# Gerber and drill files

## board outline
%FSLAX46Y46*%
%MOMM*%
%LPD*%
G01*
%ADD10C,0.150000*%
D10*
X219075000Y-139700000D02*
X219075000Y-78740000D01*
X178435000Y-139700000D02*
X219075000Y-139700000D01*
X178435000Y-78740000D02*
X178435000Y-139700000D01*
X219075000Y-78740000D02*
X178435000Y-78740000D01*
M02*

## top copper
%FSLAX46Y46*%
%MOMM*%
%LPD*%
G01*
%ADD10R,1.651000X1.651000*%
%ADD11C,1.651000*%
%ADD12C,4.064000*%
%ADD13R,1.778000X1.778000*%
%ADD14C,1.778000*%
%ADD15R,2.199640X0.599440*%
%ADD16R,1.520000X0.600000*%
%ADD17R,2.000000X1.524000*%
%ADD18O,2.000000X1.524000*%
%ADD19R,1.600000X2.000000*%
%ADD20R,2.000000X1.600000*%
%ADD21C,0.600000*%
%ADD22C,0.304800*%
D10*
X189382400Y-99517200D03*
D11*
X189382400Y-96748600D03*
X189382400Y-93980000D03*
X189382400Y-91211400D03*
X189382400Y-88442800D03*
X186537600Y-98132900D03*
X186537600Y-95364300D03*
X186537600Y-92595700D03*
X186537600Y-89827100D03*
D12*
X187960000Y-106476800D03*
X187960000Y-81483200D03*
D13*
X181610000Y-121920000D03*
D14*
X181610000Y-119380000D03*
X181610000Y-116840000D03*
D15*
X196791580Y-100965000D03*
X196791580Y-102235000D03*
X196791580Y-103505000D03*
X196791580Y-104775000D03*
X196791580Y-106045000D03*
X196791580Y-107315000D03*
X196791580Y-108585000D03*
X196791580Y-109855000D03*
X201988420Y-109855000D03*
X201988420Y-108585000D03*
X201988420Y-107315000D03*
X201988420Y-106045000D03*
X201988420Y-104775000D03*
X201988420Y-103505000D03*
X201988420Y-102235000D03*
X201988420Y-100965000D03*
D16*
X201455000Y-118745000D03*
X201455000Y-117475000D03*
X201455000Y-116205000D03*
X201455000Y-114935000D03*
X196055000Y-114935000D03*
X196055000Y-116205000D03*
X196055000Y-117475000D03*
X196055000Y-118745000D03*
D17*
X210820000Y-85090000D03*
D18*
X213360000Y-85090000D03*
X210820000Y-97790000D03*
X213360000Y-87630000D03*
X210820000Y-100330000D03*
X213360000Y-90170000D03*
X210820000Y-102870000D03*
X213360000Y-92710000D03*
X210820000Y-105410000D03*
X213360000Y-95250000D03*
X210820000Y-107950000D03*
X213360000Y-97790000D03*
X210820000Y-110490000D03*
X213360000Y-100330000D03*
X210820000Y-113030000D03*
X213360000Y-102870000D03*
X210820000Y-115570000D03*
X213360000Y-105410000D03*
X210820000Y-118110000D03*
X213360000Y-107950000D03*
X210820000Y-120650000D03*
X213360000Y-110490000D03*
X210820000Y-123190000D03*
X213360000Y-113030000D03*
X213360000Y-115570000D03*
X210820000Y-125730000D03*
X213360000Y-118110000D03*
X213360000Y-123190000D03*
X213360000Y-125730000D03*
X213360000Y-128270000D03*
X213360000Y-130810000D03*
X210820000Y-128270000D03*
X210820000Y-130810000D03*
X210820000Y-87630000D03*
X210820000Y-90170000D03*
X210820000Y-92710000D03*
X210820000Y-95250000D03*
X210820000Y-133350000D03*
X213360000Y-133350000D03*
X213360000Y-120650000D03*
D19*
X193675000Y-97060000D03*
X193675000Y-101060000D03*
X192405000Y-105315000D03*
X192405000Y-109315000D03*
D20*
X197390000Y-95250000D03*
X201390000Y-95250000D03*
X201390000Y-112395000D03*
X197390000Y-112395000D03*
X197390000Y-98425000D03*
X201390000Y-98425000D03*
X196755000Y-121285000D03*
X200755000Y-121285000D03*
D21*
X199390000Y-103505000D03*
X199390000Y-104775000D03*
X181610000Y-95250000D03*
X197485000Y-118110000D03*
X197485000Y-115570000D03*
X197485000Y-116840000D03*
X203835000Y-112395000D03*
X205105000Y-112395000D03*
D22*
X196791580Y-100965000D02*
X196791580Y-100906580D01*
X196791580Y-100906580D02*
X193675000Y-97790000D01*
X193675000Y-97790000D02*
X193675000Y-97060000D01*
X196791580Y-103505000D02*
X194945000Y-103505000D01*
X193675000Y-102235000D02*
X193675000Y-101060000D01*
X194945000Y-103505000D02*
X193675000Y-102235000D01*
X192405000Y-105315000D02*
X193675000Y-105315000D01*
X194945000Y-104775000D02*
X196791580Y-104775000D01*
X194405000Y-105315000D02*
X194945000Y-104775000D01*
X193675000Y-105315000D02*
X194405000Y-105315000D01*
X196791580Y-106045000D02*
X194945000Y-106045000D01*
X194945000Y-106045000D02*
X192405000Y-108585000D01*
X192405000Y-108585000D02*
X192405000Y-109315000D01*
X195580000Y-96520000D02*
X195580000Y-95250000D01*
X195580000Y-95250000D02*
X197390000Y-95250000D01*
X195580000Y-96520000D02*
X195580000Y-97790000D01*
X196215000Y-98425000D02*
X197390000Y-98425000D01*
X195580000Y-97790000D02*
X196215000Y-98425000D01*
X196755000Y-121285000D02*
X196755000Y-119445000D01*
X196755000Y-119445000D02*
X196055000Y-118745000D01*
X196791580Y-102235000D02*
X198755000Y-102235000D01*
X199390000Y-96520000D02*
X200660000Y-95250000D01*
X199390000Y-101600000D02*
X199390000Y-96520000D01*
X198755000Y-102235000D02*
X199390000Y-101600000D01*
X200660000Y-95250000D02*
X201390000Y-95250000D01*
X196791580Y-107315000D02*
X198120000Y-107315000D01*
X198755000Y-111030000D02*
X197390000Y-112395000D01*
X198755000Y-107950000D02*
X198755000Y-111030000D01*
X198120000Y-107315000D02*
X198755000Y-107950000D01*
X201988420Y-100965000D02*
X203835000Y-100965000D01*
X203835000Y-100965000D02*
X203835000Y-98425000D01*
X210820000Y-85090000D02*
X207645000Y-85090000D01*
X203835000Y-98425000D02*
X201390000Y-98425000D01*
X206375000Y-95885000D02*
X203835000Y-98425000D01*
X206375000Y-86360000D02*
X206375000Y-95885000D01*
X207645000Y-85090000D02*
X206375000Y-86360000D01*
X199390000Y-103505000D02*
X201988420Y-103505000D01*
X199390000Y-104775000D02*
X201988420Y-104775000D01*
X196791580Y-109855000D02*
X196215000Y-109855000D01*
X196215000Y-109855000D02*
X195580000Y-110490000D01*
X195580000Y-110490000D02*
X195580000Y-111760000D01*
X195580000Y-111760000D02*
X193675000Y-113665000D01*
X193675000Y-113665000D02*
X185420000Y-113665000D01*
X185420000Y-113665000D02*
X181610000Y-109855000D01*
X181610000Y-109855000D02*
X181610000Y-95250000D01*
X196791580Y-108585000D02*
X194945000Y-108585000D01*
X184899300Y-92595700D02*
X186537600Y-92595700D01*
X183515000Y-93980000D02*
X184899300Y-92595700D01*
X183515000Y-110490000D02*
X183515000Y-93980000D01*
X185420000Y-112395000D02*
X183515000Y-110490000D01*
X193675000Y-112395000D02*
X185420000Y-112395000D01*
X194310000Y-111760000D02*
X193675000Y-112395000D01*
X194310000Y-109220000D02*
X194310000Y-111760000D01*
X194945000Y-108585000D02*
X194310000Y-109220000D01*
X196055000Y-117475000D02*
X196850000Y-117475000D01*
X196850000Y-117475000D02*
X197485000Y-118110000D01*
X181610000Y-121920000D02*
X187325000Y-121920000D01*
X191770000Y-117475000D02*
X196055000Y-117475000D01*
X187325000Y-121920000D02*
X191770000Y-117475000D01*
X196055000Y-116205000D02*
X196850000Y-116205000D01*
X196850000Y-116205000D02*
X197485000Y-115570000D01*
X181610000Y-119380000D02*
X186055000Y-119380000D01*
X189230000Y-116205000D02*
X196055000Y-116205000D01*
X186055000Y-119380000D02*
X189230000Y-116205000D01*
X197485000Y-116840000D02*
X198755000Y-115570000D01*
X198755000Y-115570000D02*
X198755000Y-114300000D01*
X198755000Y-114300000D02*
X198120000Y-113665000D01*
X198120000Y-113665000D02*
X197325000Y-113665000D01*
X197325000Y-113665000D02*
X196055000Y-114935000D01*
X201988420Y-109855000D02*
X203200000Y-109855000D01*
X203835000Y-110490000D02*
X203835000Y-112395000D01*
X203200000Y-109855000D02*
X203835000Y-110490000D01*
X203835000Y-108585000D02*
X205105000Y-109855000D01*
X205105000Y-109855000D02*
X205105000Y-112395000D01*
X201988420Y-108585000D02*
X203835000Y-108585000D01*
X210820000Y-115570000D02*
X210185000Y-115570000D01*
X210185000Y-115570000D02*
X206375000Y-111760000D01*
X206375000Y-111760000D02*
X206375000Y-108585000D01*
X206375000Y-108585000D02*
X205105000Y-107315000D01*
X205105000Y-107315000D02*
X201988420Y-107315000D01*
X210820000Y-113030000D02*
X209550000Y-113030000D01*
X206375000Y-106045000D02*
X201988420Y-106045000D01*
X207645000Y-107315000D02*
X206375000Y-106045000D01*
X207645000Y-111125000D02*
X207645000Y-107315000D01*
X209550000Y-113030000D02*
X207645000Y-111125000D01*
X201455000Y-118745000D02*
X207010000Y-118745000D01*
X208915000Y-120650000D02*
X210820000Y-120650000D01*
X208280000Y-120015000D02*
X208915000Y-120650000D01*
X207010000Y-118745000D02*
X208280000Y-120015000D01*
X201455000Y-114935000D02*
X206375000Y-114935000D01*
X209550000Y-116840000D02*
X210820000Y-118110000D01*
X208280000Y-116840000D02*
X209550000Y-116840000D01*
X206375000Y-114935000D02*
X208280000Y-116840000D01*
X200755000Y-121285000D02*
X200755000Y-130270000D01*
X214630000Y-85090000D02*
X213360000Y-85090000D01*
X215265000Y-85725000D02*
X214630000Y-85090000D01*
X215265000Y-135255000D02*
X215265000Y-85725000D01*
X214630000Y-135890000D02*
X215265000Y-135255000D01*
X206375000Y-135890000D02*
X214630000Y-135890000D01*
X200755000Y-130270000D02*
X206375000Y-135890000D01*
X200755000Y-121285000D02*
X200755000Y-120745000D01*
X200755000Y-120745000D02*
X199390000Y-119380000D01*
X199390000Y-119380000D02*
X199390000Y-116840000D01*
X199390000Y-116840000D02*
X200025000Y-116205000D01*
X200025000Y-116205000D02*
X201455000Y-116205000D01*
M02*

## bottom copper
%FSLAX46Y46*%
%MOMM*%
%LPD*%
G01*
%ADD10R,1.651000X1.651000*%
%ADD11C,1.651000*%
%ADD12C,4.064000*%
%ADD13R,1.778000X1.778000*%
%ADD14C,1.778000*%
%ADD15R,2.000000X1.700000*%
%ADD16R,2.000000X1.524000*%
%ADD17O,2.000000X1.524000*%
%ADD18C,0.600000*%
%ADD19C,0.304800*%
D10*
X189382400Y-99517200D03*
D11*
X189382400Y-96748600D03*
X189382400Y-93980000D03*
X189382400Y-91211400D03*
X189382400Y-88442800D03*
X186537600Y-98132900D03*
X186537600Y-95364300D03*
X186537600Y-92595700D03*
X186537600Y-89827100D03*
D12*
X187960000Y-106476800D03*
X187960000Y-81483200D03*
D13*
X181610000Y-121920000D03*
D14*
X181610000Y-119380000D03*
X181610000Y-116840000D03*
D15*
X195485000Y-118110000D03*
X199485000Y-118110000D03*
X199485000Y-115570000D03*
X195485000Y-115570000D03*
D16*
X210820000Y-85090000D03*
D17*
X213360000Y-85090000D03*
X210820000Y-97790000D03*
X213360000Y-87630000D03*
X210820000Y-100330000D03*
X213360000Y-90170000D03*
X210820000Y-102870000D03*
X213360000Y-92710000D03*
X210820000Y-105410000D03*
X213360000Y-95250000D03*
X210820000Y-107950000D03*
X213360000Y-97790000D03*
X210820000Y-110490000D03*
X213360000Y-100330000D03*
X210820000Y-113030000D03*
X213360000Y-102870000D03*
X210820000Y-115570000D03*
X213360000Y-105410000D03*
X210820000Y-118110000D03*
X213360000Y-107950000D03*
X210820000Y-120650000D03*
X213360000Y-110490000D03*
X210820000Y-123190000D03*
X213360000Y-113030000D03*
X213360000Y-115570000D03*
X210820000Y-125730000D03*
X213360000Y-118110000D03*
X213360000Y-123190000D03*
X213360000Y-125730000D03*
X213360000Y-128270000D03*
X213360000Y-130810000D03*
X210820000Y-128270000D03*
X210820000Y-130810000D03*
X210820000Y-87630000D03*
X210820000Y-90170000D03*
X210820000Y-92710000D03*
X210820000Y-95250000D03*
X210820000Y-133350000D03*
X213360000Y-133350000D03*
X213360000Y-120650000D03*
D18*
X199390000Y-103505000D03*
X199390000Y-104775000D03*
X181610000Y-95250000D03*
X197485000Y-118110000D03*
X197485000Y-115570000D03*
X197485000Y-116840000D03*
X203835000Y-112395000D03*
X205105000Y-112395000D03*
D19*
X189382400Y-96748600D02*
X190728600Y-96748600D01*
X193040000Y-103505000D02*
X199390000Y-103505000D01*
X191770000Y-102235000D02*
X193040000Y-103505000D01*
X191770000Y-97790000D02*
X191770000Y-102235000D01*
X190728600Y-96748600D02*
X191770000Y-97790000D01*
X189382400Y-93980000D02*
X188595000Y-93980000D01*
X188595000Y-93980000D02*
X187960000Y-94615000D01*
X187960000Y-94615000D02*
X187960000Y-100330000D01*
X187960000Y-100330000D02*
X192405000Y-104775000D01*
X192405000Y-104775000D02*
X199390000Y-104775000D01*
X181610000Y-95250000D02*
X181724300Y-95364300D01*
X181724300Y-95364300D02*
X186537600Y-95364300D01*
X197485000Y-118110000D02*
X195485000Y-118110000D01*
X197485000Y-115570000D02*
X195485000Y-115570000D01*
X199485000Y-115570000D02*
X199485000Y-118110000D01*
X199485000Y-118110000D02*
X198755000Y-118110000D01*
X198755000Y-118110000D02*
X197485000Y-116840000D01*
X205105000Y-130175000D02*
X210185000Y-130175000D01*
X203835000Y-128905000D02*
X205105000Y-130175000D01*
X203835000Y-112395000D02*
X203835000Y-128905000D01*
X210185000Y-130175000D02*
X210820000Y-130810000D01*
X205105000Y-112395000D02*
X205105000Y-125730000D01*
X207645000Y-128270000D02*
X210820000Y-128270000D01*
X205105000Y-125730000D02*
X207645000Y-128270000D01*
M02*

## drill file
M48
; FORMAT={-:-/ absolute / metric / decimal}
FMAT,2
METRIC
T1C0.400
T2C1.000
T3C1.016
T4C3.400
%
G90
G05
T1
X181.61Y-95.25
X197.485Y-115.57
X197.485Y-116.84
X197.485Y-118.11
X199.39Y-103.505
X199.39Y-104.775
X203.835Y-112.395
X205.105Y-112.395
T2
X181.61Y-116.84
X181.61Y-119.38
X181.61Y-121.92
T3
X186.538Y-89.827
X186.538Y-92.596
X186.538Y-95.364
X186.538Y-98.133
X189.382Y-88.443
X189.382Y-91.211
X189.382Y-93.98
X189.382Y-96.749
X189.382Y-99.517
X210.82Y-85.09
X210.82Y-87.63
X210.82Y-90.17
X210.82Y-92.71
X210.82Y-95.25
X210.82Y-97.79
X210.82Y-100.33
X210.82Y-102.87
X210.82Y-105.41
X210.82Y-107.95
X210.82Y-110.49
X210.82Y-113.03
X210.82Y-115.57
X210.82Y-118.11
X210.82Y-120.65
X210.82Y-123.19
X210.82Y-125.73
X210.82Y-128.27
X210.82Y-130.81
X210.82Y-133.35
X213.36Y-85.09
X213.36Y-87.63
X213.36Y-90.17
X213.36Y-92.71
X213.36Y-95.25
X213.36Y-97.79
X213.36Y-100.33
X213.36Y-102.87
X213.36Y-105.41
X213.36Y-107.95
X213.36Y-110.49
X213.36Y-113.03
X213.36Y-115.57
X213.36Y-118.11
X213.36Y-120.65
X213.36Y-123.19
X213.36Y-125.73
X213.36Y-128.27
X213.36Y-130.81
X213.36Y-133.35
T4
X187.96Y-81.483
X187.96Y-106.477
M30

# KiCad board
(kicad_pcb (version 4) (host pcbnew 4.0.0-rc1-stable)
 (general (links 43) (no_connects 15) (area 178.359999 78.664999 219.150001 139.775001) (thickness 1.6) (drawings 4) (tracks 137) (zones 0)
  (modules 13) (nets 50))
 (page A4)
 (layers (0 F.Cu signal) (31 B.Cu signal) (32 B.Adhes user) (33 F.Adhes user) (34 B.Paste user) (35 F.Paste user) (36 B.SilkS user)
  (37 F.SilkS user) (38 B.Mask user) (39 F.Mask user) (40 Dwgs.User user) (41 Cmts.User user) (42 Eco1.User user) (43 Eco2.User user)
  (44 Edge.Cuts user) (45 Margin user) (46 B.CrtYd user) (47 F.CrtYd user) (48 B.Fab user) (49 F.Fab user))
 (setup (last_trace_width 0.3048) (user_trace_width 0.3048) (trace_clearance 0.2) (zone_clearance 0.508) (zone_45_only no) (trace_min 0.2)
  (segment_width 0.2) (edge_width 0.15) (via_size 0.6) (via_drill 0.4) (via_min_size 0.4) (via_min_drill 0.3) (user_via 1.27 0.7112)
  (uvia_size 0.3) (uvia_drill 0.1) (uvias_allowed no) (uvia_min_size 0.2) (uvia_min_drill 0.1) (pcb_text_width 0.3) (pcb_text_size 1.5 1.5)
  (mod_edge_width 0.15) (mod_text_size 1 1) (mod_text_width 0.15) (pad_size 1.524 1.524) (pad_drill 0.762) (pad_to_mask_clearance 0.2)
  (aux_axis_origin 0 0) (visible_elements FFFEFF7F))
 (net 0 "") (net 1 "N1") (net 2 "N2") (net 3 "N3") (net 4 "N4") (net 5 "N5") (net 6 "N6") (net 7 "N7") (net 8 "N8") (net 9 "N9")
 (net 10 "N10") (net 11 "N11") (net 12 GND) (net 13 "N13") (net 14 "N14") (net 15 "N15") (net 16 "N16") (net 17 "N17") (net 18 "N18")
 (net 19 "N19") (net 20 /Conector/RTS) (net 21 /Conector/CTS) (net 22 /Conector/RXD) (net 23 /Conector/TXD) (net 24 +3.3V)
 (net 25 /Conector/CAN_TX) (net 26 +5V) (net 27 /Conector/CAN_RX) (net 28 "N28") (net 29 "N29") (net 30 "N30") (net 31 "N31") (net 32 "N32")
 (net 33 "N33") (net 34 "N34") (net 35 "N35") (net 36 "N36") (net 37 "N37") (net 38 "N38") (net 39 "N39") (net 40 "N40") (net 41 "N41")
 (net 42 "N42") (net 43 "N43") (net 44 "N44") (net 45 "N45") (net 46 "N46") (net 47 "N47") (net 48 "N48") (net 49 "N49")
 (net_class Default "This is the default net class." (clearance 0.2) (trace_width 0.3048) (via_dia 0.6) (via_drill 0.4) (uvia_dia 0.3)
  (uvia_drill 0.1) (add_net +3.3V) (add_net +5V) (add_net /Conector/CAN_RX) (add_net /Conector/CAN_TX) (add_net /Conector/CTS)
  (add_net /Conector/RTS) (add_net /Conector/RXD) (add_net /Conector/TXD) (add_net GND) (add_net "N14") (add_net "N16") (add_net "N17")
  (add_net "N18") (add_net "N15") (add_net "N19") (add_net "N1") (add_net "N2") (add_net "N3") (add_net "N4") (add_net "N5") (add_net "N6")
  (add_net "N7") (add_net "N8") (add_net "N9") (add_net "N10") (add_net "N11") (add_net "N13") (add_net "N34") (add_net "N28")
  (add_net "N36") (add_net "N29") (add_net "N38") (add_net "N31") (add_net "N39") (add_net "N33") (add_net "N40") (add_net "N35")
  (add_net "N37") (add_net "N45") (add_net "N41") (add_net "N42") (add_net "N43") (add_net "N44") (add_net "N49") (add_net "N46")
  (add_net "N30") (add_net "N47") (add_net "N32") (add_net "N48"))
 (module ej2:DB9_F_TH (layer F.Cu) (at 187.96 93.98 90)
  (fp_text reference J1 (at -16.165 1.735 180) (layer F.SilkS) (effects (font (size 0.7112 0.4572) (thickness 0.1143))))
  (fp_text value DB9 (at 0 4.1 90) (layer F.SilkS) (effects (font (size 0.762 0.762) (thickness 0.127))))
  (pad 1 thru_hole rect (at -5.5372 1.4224 90) (size 1.651 1.651) (drill 1.016) (layers *.Cu *.Mask) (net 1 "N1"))
  (pad 2 thru_hole circle (at -2.7686 1.4224 90) (size 1.651 1.651) (drill 1.016) (layers *.Cu *.Mask) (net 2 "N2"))
  (pad 3 thru_hole circle (at 0 1.4224 90) (size 1.651 1.651) (drill 1.016) (layers *.Cu *.Mask) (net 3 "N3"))
  (pad 4 thru_hole circle (at 2.7686 1.4224 90) (size 1.651 1.651) (drill 1.016) (layers *.Cu *.Mask) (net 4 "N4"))
  (pad 5 thru_hole circle (at 5.5372 1.4224 90) (size 1.651 1.651) (drill 1.016) (layers *.Cu *.Mask) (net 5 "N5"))
  (pad 6 thru_hole circle (at -4.1529 -1.4224 90) (size 1.651 1.651) (drill 1.016) (layers *.Cu *.Mask) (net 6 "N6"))
  (pad 7 thru_hole circle (at -1.3843 -1.4224 90) (size 1.651 1.651) (drill 1.016) (layers *.Cu *.Mask) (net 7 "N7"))
  (pad 8 thru_hole circle (at 1.3843 -1.4224 90) (size 1.651 1.651) (drill 1.016) (layers *.Cu *.Mask) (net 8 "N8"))
  (pad 9 thru_hole circle (at 4.1529 -1.4224 90) (size 1.651 1.651) (drill 1.016) (layers *.Cu *.Mask) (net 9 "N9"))
  (pad 10 thru_hole circle (at -12.4968 0 90) (size 4.064 4.064) (drill 3.4) (layers *.Cu *.Mask))
  (pad 11 thru_hole circle (at 12.4968 0 90) (size 4.064 4.064) (drill 3.4) (layers *.Cu *.Mask)))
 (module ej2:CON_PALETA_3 (layer F.Cu) (at 181.61 119.38 90)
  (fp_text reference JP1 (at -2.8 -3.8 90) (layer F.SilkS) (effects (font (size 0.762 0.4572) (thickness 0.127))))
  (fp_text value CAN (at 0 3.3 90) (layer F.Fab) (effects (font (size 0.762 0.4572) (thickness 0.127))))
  (pad 1 thru_hole rect (at -2.54 0 90) (size 1.778 1.778) (drill 1) (layers *.Cu *.Mask) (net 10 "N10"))
  (pad 2 thru_hole circle (at 0 0 90) (size 1.778 1.778) (drill 1) (layers *.Cu *.Mask) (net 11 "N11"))
  (pad 3 thru_hole circle (at 2.54 0 90) (size 1.778 1.778) (drill 1) (layers *.Cu *.Mask) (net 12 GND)))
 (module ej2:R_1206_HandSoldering (layer B.Cu) (at 197.485 118.11)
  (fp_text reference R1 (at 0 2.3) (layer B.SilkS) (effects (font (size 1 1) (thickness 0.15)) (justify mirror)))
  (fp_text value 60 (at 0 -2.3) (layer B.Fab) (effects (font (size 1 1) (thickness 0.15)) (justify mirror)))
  (pad 1 smd rect (at -2 0) (size 2 1.7) (layers B.Cu B.Paste B.Mask) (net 10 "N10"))
  (pad 2 smd rect (at 2 0) (size 2 1.7) (layers B.Cu B.Paste B.Mask) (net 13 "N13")))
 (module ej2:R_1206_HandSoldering (layer B.Cu) (at 197.485 115.57 180)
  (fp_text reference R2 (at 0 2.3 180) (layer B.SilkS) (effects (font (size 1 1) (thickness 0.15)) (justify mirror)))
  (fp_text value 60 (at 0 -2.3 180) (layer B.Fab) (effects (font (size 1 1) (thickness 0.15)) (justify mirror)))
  (pad 1 smd rect (at -2 0 180) (size 2 1.7) (layers B.Cu B.Paste B.Mask) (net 13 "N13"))
  (pad 2 smd rect (at 2 0 180) (size 2 1.7) (layers B.Cu B.Paste B.Mask) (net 11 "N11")))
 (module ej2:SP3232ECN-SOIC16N (layer F.Cu) (at 199.39 105.41 270)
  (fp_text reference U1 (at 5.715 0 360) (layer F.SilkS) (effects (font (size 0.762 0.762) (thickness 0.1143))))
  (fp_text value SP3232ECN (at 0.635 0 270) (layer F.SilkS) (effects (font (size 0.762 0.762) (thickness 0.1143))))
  (pad 1 smd rect (at -4.445 2.59842 270) (size 0.59944 2.19964) (layers F.Cu F.Paste F.Mask) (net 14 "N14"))
  (pad 2 smd rect (at -3.175 2.59842 270) (size 0.59944 2.19964) (layers F.Cu F.Paste F.Mask) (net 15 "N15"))
  (pad 3 smd rect (at -1.905 2.59842 270) (size 0.59944 2.19964) (layers F.Cu F.Paste F.Mask) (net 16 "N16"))
  (pad 4 smd rect (at -0.635 2.59842 270) (size 0.59944 2.19964) (layers F.Cu F.Paste F.Mask) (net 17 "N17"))
  (pad 5 smd rect (at 0.635 2.59842 270) (size 0.59944 2.19964) (layers F.Cu F.Paste F.Mask) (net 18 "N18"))
  (pad 6 smd rect (at 1.905 2.59842 270) (size 0.59944 2.19964) (layers F.Cu F.Paste F.Mask) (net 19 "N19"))
  (pad 7 smd rect (at 3.175 2.59842 270) (size 0.59944 2.19964) (layers F.Cu F.Paste F.Mask) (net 8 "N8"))
  (pad 8 smd rect (at 4.445 2.59842 270) (size 0.59944 2.19964) (layers F.Cu F.Paste F.Mask) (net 7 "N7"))
  (pad 9 smd rect (at 4.445 -2.59842 270) (size 0.59944 2.19964) (layers F.Cu F.Paste F.Mask) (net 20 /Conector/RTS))
  (pad 10 smd rect (at 3.175 -2.59842 270) (size 0.59944 2.19964) (layers F.Cu F.Paste F.Mask) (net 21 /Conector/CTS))
  (pad 11 smd rect (at 1.905 -2.59842 270) (size 0.59944 2.19964) (layers F.Cu F.Paste F.Mask) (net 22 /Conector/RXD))
  (pad 12 smd rect (at 0.635 -2.59842 270) (size 0.59944 2.19964) (layers F.Cu F.Paste F.Mask) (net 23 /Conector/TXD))
  (pad 13 smd rect (at -0.635 -2.59842 270) (size 0.59944 2.19964) (layers F.Cu F.Paste F.Mask) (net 3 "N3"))
  (pad 14 smd rect (at -1.905 -2.59842 270) (size 0.59944 2.19964) (layers F.Cu F.Paste F.Mask) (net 2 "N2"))
  (pad 15 smd rect (at -3.175 -2.59842 270) (size 0.59944 2.19964) (layers F.Cu F.Paste F.Mask) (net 12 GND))
  (pad 16 smd rect (at -4.445 -2.59842 270) (size 0.59944 2.19964) (layers F.Cu F.Paste F.Mask) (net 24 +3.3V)))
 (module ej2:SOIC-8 (layer F.Cu) (at 198.755 116.84 180)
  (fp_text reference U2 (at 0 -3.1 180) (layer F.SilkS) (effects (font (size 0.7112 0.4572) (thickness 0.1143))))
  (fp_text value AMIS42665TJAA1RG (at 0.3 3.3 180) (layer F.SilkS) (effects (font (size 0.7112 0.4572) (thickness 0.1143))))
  (pad 1 smd rect (at -2.7 -1.905 90) (size 0.6 1.52) (layers F.Cu F.Paste F.Mask) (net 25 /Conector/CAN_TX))
  (pad 2 smd rect (at -2.7 -0.635 90) (size 0.6 1.52) (layers F.Cu F.Paste F.Mask) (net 12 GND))
  (pad 3 smd rect (at -2.7 0.635 90) (size 0.6 1.52) (layers F.Cu F.Paste F.Mask) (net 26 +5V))
  (pad 4 smd rect (at -2.7 1.905 90) (size 0.6 1.52) (layers F.Cu F.Paste F.Mask) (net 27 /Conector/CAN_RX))
  (pad 5 smd rect (at 2.7 1.905 90) (size 0.6 1.52) (layers F.Cu F.Paste F.Mask) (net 13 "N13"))
  (pad 6 smd rect (at 2.7 0.635 90) (size 0.6 1.52) (layers F.Cu F.Paste F.Mask) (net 11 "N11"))
  (pad 7 smd rect (at 2.7 -0.635 90) (size 0.6 1.52) (layers F.Cu F.Paste F.Mask) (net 10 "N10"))
  (pad 8 smd rect (at 2.7 -1.905 90) (size 0.6 1.52) (layers F.Cu F.Paste F.Mask) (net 12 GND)))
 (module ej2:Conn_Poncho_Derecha (layer F.Cu) (at 210.82 85.09)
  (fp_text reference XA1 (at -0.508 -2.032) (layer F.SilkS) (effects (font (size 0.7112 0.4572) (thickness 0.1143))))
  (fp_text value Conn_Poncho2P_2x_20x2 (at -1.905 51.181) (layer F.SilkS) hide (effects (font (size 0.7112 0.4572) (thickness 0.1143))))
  (pad 1 thru_hole rect (at 0 0 270) (size 1.524 2) (drill 1.016) (layers *.Cu *.Mask) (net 24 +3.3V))
  (pad 2 thru_hole oval (at 2.54 0 270) (size 1.524 2) (drill 1.016) (layers *.Cu *.Mask) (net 26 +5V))
  (pad 11 thru_hole oval (at 0 12.7 270) (size 1.524 2) (drill 1.016) (layers *.Cu *.Mask) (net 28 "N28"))
  (pad 4 thru_hole oval (at 2.54 2.54 270) (size 1.524 2) (drill 1.016) (layers *.Cu *.Mask) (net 12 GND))
  (pad 13 thru_hole oval (at 0 15.24 270) (size 1.524 2) (drill 1.016) (layers *.Cu *.Mask) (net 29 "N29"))
  (pad 6 thru_hole oval (at 2.54 5.08 270) (size 1.524 2) (drill 1.016) (layers *.Cu *.Mask) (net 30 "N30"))
  (pad 15 thru_hole oval (at 0 17.78 270) (size 1.524 2) (drill 1.016) (layers *.Cu *.Mask) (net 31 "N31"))
  (pad 8 thru_hole oval (at 2.54 7.62 270) (size 1.524 2) (drill 1.016) (layers *.Cu *.Mask) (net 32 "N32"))
  (pad 17 thru_hole oval (at 0 20.32 270) (size 1.524 2) (drill 1.016) (layers *.Cu *.Mask) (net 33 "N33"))
  (pad 10 thru_hole oval (at 2.54 10.16 270) (size 1.524 2) (drill 1.016) (layers *.Cu *.Mask) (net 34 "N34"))
  (pad 19 thru_hole oval (at 0 22.86 270) (size 1.524 2) (drill 1.016) (layers *.Cu *.Mask) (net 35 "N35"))
  (pad 12 thru_hole oval (at 2.54 12.7 270) (size 1.524 2) (drill 1.016) (layers *.Cu *.Mask) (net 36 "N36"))
  (pad 21 thru_hole oval (at 0 25.4 270) (size 1.524 2) (drill 1.016) (layers *.Cu *.Mask) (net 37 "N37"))
  (pad 14 thru_hole oval (at 2.54 15.24 270) (size 1.524 2) (drill 1.016) (layers *.Cu *.Mask) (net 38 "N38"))
  (pad 23 thru_hole oval (at 0 27.94 270) (size 1.524 2) (drill 1.016) (layers *.Cu *.Mask) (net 23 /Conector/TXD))
  (pad 16 thru_hole oval (at 2.54 17.78 270) (size 1.524 2) (drill 1.016) (layers *.Cu *.Mask) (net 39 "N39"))
  (pad 25 thru_hole oval (at 0 30.48 270) (size 1.524 2) (drill 1.016) (layers *.Cu *.Mask) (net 22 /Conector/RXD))
  (pad 18 thru_hole oval (at 2.54 20.32 270) (size 1.524 2) (drill 1.016) (layers *.Cu *.Mask) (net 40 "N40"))
  (pad 27 thru_hole oval (at 0 33.02 270) (size 1.524 2) (drill 1.016) (layers *.Cu *.Mask) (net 27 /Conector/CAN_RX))
  (pad 20 thru_hole oval (at 2.54 22.86 270) (size 1.524 2) (drill 1.016) (layers *.Cu *.Mask) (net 12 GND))
  (pad 29 thru_hole oval (at 0 35.56 270) (size 1.524 2) (drill 1.016) (layers *.Cu *.Mask) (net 25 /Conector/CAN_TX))
  (pad 22 thru_hole oval (at 2.54 25.4 270) (size 1.524 2) (drill 1.016) (layers *.Cu *.Mask) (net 12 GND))
  (pad 31 thru_hole oval (at 0 38.1 270) (size 1.524 2) (drill 1.016) (layers *.Cu *.Mask) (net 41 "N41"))
  (pad 24 thru_hole oval (at 2.54 27.94 270) (size 1.524 2) (drill 1.016) (layers *.Cu *.Mask) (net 12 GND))
  (pad 26 thru_hole oval (at 2.54 30.48 270) (size 1.524 2) (drill 1.016) (layers *.Cu *.Mask) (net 12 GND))
  (pad 33 thru_hole oval (at 0 40.64 270) (size 1.524 2) (drill 1.016) (layers *.Cu *.Mask) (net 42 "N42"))
  (pad 28 thru_hole oval (at 2.54 33.02 270) (size 1.524 2) (drill 1.016) (layers *.Cu *.Mask) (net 12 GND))
  (pad 32 thru_hole oval (at 2.54 38.1 270) (size 1.524 2) (drill 1.016) (layers *.Cu *.Mask) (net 12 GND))
  (pad 34 thru_hole oval (at 2.54 40.64 270) (size 1.524 2) (drill 1.016) (layers *.Cu *.Mask) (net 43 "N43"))
  (pad 36 thru_hole oval (at 2.54 43.18 270) (size 1.524 2) (drill 1.016) (layers *.Cu *.Mask) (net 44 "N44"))
  (pad 38 thru_hole oval (at 2.54 45.72 270) (size 1.524 2) (drill 1.016) (layers *.Cu *.Mask) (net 12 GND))
  (pad 35 thru_hole oval (at 0 43.18 270) (size 1.524 2) (drill 1.016) (layers *.Cu *.Mask) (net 21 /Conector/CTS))
  (pad 37 thru_hole oval (at 0 45.72 270) (size 1.524 2) (drill 1.016) (layers *.Cu *.Mask) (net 20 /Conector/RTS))
  (pad 3 thru_hole oval (at 0 2.54 270) (size 1.524 2) (drill 1.016) (layers *.Cu *.Mask) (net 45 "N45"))
  (pad 5 thru_hole oval (at 0 5.08 270) (size 1.524 2) (drill 1.016) (layers *.Cu *.Mask) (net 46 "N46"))
  (pad 7 thru_hole oval (at 0 7.62 270) (size 1.524 2) (drill 1.016) (layers *.Cu *.Mask) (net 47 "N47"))
  (pad 9 thru_hole oval (at 0 10.16 270) (size 1.524 2) (drill 1.016) (layers *.Cu *.Mask) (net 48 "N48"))
  (pad 39 thru_hole oval (at 0 48.26 270) (size 1.524 2) (drill 1.016) (layers *.Cu *.Mask) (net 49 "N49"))
  (pad 40 thru_hole oval (at 2.54 48.26 270) (size 1.524 2) (drill 1.016) (layers *.Cu *.Mask) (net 12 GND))
  (pad 30 thru_hole oval (at 2.54 35.56 270) (size 1.524 2) (drill 1.016) (layers *.Cu *.Mask) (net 12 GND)))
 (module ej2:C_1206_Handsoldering (layer F.Cu) (at 193.675 99.06 270)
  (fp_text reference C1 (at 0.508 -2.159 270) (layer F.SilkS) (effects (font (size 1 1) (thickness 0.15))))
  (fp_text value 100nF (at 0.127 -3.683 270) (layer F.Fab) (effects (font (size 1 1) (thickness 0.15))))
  (pad 1 smd rect (at -2 0 270) (size 2 1.6) (layers F.Cu F.Paste F.Mask) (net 14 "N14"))
  (pad 2 smd rect (at 2 0 270) (size 2 1.6) (layers F.Cu F.Paste F.Mask) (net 16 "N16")))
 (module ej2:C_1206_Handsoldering (layer F.Cu) (at 192.405 107.315 270)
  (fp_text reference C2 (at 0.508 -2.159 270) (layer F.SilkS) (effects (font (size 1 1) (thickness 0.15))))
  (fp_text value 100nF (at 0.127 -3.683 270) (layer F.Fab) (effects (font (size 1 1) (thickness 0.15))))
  (pad 1 smd rect (at -2 0 270) (size 2 1.6) (layers F.Cu F.Paste F.Mask) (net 17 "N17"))
  (pad 2 smd rect (at 2 0 270) (size 2 1.6) (layers F.Cu F.Paste F.Mask) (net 18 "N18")))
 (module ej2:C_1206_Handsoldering (layer F.Cu) (at 199.39 95.25)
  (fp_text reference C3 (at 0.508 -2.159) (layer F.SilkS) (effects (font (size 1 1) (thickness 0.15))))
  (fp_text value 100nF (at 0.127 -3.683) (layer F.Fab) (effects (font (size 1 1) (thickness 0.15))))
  (pad 1 smd rect (at -2 0) (size 2 1.6) (layers F.Cu F.Paste F.Mask) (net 12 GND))
  (pad 2 smd rect (at 2 0) (size 2 1.6) (layers F.Cu F.Paste F.Mask) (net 15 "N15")))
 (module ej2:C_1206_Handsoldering (layer F.Cu) (at 199.39 112.395 180)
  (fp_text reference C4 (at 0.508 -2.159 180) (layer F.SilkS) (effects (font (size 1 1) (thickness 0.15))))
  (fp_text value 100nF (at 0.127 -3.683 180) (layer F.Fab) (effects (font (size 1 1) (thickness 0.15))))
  (pad 1 smd rect (at -2 0 180) (size 2 1.6) (layers F.Cu F.Paste F.Mask) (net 12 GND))
  (pad 2 smd rect (at 2 0 180) (size 2 1.6) (layers F.Cu F.Paste F.Mask) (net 19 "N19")))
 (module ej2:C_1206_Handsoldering (layer F.Cu) (at 199.39 98.425)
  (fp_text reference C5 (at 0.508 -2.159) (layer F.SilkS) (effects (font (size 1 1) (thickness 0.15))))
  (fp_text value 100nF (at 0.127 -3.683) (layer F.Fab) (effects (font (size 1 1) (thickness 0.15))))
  (pad 1 smd rect (at -2 0) (size 2 1.6) (layers F.Cu F.Paste F.Mask) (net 12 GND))
  (pad 2 smd rect (at 2 0) (size 2 1.6) (layers F.Cu F.Paste F.Mask) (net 24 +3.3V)))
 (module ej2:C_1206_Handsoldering (layer F.Cu) (at 198.755 121.285)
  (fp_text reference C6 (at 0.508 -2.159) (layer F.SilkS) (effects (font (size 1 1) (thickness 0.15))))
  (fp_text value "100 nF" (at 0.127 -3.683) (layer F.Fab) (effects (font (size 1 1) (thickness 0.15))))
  (pad 1 smd rect (at -2 0) (size 2 1.6) (layers F.Cu F.Paste F.Mask) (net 12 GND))
  (pad 2 smd rect (at 2 0) (size 2 1.6) (layers F.Cu F.Paste F.Mask) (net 26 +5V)))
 (gr_line (start 219.075 139.7) (end 219.075 78.74) (angle 90) (layer Edge.Cuts) (width 0.15))
 (gr_line (start 178.435 139.7) (end 219.075 139.7) (angle 90) (layer Edge.Cuts) (width 0.15))
 (gr_line (start 178.435 78.74) (end 178.435 139.7) (angle 90) (layer Edge.Cuts) (width 0.15))
 (gr_line (start 219.075 78.74) (end 178.435 78.74) (angle 90) (layer Edge.Cuts) (width 0.15))
 (segment (start 196.79158 100.965) (end 196.79158 100.90658) (width 0.3048) (layer F.Cu) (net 14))
 (segment (start 196.79158 100.90658) (end 193.675 97.79) (width 0.3048) (layer F.Cu) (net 14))
 (segment (start 193.675 97.79) (end 193.675 97.06) (width 0.3048) (layer F.Cu) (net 14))
 (segment (start 196.79158 103.505) (end 194.945 103.505) (width 0.3048) (layer F.Cu) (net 16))
 (segment (start 193.675 102.235) (end 193.675 101.06) (width 0.3048) (layer F.Cu) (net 16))
 (segment (start 194.945 103.505) (end 193.675 102.235) (width 0.3048) (layer F.Cu) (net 16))
 (segment (start 192.405 105.315) (end 193.675 105.315) (width 0.3048) (layer F.Cu) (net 17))
 (segment (start 194.945 104.775) (end 196.79158 104.775) (width 0.3048) (layer F.Cu) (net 17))
 (segment (start 194.405 105.315) (end 194.945 104.775) (width 0.3048) (layer F.Cu) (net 17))
 (segment (start 193.675 105.315) (end 194.405 105.315) (width 0.3048) (layer F.Cu) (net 17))
 (segment (start 196.79158 106.045) (end 194.945 106.045) (width 0.3048) (layer F.Cu) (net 18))
 (segment (start 194.945 106.045) (end 192.405 108.585) (width 0.3048) (layer F.Cu) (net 18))
 (segment (start 192.405 108.585) (end 192.405 109.315) (width 0.3048) (layer F.Cu) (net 18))
 (segment (start 195.58 96.52) (end 195.58 95.25) (width 0.3048) (layer F.Cu) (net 12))
 (segment (start 195.58 95.25) (end 197.39 95.25) (width 0.3048) (layer F.Cu) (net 12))
 (segment (start 195.58 96.52) (end 195.58 97.79) (width 0.3048) (layer F.Cu) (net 12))
 (segment (start 196.215 98.425) (end 197.39 98.425) (width 0.3048) (layer F.Cu) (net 12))
 (segment (start 195.58 97.79) (end 196.215 98.425) (width 0.3048) (layer F.Cu) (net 12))
 (segment (start 196.755 121.285) (end 196.755 119.445) (width 0.3048) (layer F.Cu) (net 12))
 (segment (start 196.755 119.445) (end 196.055 118.745) (width 0.3048) (layer F.Cu) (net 12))
 (segment (start 196.79158 102.235) (end 198.755 102.235) (width 0.3048) (layer F.Cu) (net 15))
 (segment (start 199.39 96.52) (end 200.66 95.25) (width 0.3048) (layer F.Cu) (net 15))
 (segment (start 199.39 101.6) (end 199.39 96.52) (width 0.3048) (layer F.Cu) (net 15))
 (segment (start 198.755 102.235) (end 199.39 101.6) (width 0.3048) (layer F.Cu) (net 15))
 (segment (start 200.66 95.25) (end 201.39 95.25) (width 0.3048) (layer F.Cu) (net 15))
 (segment (start 196.79158 107.315) (end 198.12 107.315) (width 0.3048) (layer F.Cu) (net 19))
 (segment (start 198.755 111.03) (end 197.39 112.395) (width 0.3048) (layer F.Cu) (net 19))
 (segment (start 198.755 107.95) (end 198.755 111.03) (width 0.3048) (layer F.Cu) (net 19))
 (segment (start 198.12 107.315) (end 198.755 107.95) (width 0.3048) (layer F.Cu) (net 19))
 (segment (start 201.98842 100.965) (end 203.835 100.965) (width 0.3048) (layer F.Cu) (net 24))
 (segment (start 203.835 100.965) (end 203.835 98.425) (width 0.3048) (layer F.Cu) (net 24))
 (segment (start 210.82 85.09) (end 207.645 85.09) (width 0.3048) (layer F.Cu) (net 24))
 (segment (start 203.835 98.425) (end 201.39 98.425) (width 0.3048) (layer F.Cu) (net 24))
 (segment (start 206.375 95.885) (end 203.835 98.425) (width 0.3048) (layer F.Cu) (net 24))
 (segment (start 206.375 86.36) (end 206.375 95.885) (width 0.3048) (layer F.Cu) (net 24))
 (segment (start 207.645 85.09) (end 206.375 86.36) (width 0.3048) (layer F.Cu) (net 24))
 (segment (start 189.3824 96.7486) (end 190.7286 96.7486) (width 0.3048) (layer B.Cu) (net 2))
 (segment (start 199.39 103.505) (end 201.98842 103.505) (width 0.3048) (layer F.Cu) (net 2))
 (via (at 199.39 103.505) (size 0.6) (drill 0.4) (layers F.Cu B.Cu) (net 2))
 (segment (start 193.04 103.505) (end 199.39 103.505) (width 0.3048) (layer B.Cu) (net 2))
 (segment (start 191.77 102.235) (end 193.04 103.505) (width 0.3048) (layer B.Cu) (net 2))
 (segment (start 191.77 97.79) (end 191.77 102.235) (width 0.3048) (layer B.Cu) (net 2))
 (segment (start 190.7286 96.7486) (end 191.77 97.79) (width 0.3048) (layer B.Cu) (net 2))
 (segment (start 189.3824 93.98) (end 188.595 93.98) (width 0.3048) (layer B.Cu) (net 3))
 (segment (start 188.595 93.98) (end 187.96 94.615) (width 0.3048) (layer B.Cu) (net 3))
 (segment (start 187.96 94.615) (end 187.96 100.33) (width 0.3048) (layer B.Cu) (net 3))
 (segment (start 187.96 100.33) (end 192.405 104.775) (width 0.3048) (layer B.Cu) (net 3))
 (segment (start 192.405 104.775) (end 199.39 104.775) (width 0.3048) (layer B.Cu) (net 3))
 (via (at 199.39 104.775) (size 0.6) (drill 0.4) (layers F.Cu B.Cu) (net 3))
 (segment (start 199.39 104.775) (end 201.98842 104.775) (width 0.3048) (layer F.Cu) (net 3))
 (segment (start 196.79158 109.855) (end 196.215 109.855) (width 0.3048) (layer F.Cu) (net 7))
 (segment (start 196.215 109.855) (end 195.58 110.49) (width 0.3048) (layer F.Cu) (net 7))
 (segment (start 195.58 110.49) (end 195.58 111.76) (width 0.3048) (layer F.Cu) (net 7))
 (segment (start 195.58 111.76) (end 193.675 113.665) (width 0.3048) (layer F.Cu) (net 7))
 (segment (start 193.675 113.665) (end 185.42 113.665) (width 0.3048) (layer F.Cu) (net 7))
 (segment (start 185.42 113.665) (end 181.61 109.855) (width 0.3048) (layer F.Cu) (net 7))
 (segment (start 181.61 109.855) (end 181.61 95.25) (width 0.3048) (layer F.Cu) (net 7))
 (via (at 181.61 95.25) (size 0.6) (drill 0.4) (layers F.Cu B.Cu) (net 7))
 (segment (start 181.61 95.25) (end 181.7243 95.3643) (width 0.3048) (layer B.Cu) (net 7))
 (segment (start 181.7243 95.3643) (end 186.5376 95.3643) (width 0.3048) (layer B.Cu) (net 7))
 (segment (start 196.79158 108.585) (end 194.945 108.585) (width 0.3048) (layer F.Cu) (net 8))
 (segment (start 184.8993 92.5957) (end 186.5376 92.5957) (width 0.3048) (layer F.Cu) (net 8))
 (segment (start 183.515 93.98) (end 184.8993 92.5957) (width 0.3048) (layer F.Cu) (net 8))
 (segment (start 183.515 110.49) (end 183.515 93.98) (width 0.3048) (layer F.Cu) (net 8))
 (segment (start 185.42 112.395) (end 183.515 110.49) (width 0.3048) (layer F.Cu) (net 8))
 (segment (start 193.675 112.395) (end 185.42 112.395) (width 0.3048) (layer F.Cu) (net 8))
 (segment (start 194.31 111.76) (end 193.675 112.395) (width 0.3048) (layer F.Cu) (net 8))
 (segment (start 194.31 109.22) (end 194.31 111.76) (width 0.3048) (layer F.Cu) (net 8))
 (segment (start 194.945 108.585) (end 194.31 109.22) (width 0.3048) (layer F.Cu) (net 8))
 (segment (start 196.055 117.475) (end 196.85 117.475) (width 0.3048) (layer F.Cu) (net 10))
 (segment (start 197.485 118.11) (end 195.485 118.11) (width 0.3048) (layer B.Cu) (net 10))
 (via (at 197.485 118.11) (size 0.6) (drill 0.4) (layers F.Cu B.Cu) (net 10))
 (segment (start 196.85 117.475) (end 197.485 118.11) (width 0.3048) (layer F.Cu) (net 10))
 (segment (start 181.61 121.92) (end 187.325 121.92) (width 0.3048) (layer F.Cu) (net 10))
 (segment (start 191.77 117.475) (end 196.055 117.475) (width 0.3048) (layer F.Cu) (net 10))
 (segment (start 187.325 121.92) (end 191.77 117.475) (width 0.3048) (layer F.Cu) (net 10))
 (segment (start 196.055 116.205) (end 196.85 116.205) (width 0.3048) (layer F.Cu) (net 11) (status 400000))
 (segment (start 197.485 115.57) (end 195.485 115.57) (width 0.3048) (layer B.Cu) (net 11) (status 800000))
 (via (at 197.485 115.57) (size 0.6) (drill 0.4) (layers F.Cu B.Cu) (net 11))
 (segment (start 196.85 116.205) (end 197.485 115.57) (width 0.3048) (layer F.Cu) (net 11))
 (segment (start 181.61 119.38) (end 186.055 119.38) (width 0.3048) (layer F.Cu) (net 11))
 (segment (start 189.23 116.205) (end 196.055 116.205) (width 0.3048) (layer F.Cu) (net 11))
 (segment (start 186.055 119.38) (end 189.23 116.205) (width 0.3048) (layer F.Cu) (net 11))
 (segment (start 199.485 115.57) (end 199.485 118.11) (width 0.3048) (layer B.Cu) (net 13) (status C00000))
 (segment (start 199.485 118.11) (end 198.755 118.11) (width 0.3048) (layer B.Cu) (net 13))
 (segment (start 198.755 118.11) (end 197.485 116.84) (width 0.3048) (layer B.Cu) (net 13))
 (via (at 197.485 116.84) (size 0.6) (drill 0.4) (layers F.Cu B.Cu) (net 13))
 (segment (start 197.485 116.84) (end 198.755 115.57) (width 0.3048) (layer F.Cu) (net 13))
 (segment (start 198.755 115.57) (end 198.755 114.3) (width 0.3048) (layer F.Cu) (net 13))
 (segment (start 198.755 114.3) (end 198.12 113.665) (width 0.3048) (layer F.Cu) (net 13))
 (segment (start 198.12 113.665) (end 197.325 113.665) (width 0.3048) (layer F.Cu) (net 13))
 (segment (start 197.325 113.665) (end 196.055 114.935) (width 0.3048) (layer F.Cu) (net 13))
 (segment (start 201.98842 109.855) (end 203.2 109.855) (width 0.3048) (layer F.Cu) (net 20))
 (segment (start 205.105 130.175) (end 210.185 130.175) (width 0.3048) (layer B.Cu) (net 20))
 (segment (start 203.835 128.905) (end 205.105 130.175) (width 0.3048) (layer B.Cu) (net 20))
 (segment (start 203.835 112.395) (end 203.835 128.905) (width 0.3048) (layer B.Cu) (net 20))
 (via (at 203.835 112.395) (size 0.6) (drill 0.4) (layers F.Cu B.Cu) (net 20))
 (segment (start 203.835 110.49) (end 203.835 112.395) (width 0.3048) (layer F.Cu) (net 20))
 (segment (start 203.2 109.855) (end 203.835 110.49) (width 0.3048) (layer F.Cu) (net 20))
 (segment (start 210.185 130.175) (end 210.82 130.81) (width 0.3048) (layer B.Cu) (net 20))
 (segment (start 205.105 112.395) (end 205.105 125.73) (width 0.3048) (layer B.Cu) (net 21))
 (segment (start 203.835 108.585) (end 205.105 109.855) (width 0.3048) (layer F.Cu) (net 21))
 (segment (start 205.105 109.855) (end 205.105 112.395) (width 0.3048) (layer F.Cu) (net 21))
 (via (at 205.105 112.395) (size 0.6) (drill 0.4) (layers F.Cu B.Cu) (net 21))
 (segment (start 201.98842 108.585) (end 203.835 108.585) (width 0.3048) (layer F.Cu) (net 21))
 (segment (start 207.645 128.27) (end 210.82 128.27) (width 0.3048) (layer B.Cu) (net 21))
 (segment (start 205.105 125.73) (end 207.645 128.27) (width 0.3048) (layer B.Cu) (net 21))
 (segment (start 210.82 115.57) (end 210.185 115.57) (width 0.3048) (layer F.Cu) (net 22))
 (segment (start 210.185 115.57) (end 206.375 111.76) (width 0.3048) (layer F.Cu) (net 22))
 (segment (start 206.375 111.76) (end 206.375 108.585) (width 0.3048) (layer F.Cu) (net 22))
 (segment (start 206.375 108.585) (end 205.105 107.315) (width 0.3048) (layer F.Cu) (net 22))
 (segment (start 205.105 107.315) (end 201.98842 107.315) (width 0.3048) (layer F.Cu) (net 22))
 (segment (start 210.82 113.03) (end 209.55 113.03) (width 0.3048) (layer F.Cu) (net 23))
 (segment (start 206.375 106.045) (end 201.98842 106.045) (width 0.3048) (layer F.Cu) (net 23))
 (segment (start 207.645 107.315) (end 206.375 106.045) (width 0.3048) (layer F.Cu) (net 23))
 (segment (start 207.645 111.125) (end 207.645 107.315) (width 0.3048) (layer F.Cu) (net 23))
 (segment (start 209.55 113.03) (end 207.645 111.125) (width 0.3048) (layer F.Cu) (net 23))
 (segment (start 201.455 118.745) (end 207.01 118.745) (width 0.3048) (layer F.Cu) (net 25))
 (segment (start 208.915 120.65) (end 210.82 120.65) (width 0.3048) (layer F.Cu) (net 25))
 (segment (start 208.28 120.015) (end 208.915 120.65) (width 0.3048) (layer F.Cu) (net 25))
 (segment (start 207.01 118.745) (end 208.28 120.015) (width 0.3048) (layer F.Cu) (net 25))
 (segment (start 201.455 114.935) (end 206.375 114.935) (width 0.3048) (layer F.Cu) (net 27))
 (segment (start 209.55 116.84) (end 210.82 118.11) (width 0.3048) (layer F.Cu) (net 27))
 (segment (start 208.28 116.84) (end 209.55 116.84) (width 0.3048) (layer F.Cu) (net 27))
 (segment (start 206.375 114.935) (end 208.28 116.84) (width 0.3048) (layer F.Cu) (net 27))
 (segment (start 200.755 121.285) (end 200.755 130.27) (width 0.3048) (layer F.Cu) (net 26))
 (segment (start 214.63 85.09) (end 213.36 85.09) (width 0.3048) (layer F.Cu) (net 26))
 (segment (start 215.265 85.725) (end 214.63 85.09) (width 0.3048) (layer F.Cu) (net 26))
 (segment (start 215.265 135.255) (end 215.265 85.725) (width 0.3048) (layer F.Cu) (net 26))
 (segment (start 214.63 135.89) (end 215.265 135.255) (width 0.3048) (layer F.Cu) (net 26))
 (segment (start 206.375 135.89) (end 214.63 135.89) (width 0.3048) (layer F.Cu) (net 26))
 (segment (start 200.755 130.27) (end 206.375 135.89) (width 0.3048) (layer F.Cu) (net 26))
 (segment (start 200.755 121.285) (end 200.755 120.745) (width 0.3048) (layer F.Cu) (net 26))
 (segment (start 200.755 120.745) (end 199.39 119.38) (width 0.3048) (layer F.Cu) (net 26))
 (segment (start 199.39 119.38) (end 199.39 116.84) (width 0.3048) (layer F.Cu) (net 26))
 (segment (start 199.39 116.84) (end 200.025 116.205) (width 0.3048) (layer F.Cu) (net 26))
 (segment (start 200.025 116.205) (end 201.455 116.205) (width 0.3048) (layer F.Cu) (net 26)))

